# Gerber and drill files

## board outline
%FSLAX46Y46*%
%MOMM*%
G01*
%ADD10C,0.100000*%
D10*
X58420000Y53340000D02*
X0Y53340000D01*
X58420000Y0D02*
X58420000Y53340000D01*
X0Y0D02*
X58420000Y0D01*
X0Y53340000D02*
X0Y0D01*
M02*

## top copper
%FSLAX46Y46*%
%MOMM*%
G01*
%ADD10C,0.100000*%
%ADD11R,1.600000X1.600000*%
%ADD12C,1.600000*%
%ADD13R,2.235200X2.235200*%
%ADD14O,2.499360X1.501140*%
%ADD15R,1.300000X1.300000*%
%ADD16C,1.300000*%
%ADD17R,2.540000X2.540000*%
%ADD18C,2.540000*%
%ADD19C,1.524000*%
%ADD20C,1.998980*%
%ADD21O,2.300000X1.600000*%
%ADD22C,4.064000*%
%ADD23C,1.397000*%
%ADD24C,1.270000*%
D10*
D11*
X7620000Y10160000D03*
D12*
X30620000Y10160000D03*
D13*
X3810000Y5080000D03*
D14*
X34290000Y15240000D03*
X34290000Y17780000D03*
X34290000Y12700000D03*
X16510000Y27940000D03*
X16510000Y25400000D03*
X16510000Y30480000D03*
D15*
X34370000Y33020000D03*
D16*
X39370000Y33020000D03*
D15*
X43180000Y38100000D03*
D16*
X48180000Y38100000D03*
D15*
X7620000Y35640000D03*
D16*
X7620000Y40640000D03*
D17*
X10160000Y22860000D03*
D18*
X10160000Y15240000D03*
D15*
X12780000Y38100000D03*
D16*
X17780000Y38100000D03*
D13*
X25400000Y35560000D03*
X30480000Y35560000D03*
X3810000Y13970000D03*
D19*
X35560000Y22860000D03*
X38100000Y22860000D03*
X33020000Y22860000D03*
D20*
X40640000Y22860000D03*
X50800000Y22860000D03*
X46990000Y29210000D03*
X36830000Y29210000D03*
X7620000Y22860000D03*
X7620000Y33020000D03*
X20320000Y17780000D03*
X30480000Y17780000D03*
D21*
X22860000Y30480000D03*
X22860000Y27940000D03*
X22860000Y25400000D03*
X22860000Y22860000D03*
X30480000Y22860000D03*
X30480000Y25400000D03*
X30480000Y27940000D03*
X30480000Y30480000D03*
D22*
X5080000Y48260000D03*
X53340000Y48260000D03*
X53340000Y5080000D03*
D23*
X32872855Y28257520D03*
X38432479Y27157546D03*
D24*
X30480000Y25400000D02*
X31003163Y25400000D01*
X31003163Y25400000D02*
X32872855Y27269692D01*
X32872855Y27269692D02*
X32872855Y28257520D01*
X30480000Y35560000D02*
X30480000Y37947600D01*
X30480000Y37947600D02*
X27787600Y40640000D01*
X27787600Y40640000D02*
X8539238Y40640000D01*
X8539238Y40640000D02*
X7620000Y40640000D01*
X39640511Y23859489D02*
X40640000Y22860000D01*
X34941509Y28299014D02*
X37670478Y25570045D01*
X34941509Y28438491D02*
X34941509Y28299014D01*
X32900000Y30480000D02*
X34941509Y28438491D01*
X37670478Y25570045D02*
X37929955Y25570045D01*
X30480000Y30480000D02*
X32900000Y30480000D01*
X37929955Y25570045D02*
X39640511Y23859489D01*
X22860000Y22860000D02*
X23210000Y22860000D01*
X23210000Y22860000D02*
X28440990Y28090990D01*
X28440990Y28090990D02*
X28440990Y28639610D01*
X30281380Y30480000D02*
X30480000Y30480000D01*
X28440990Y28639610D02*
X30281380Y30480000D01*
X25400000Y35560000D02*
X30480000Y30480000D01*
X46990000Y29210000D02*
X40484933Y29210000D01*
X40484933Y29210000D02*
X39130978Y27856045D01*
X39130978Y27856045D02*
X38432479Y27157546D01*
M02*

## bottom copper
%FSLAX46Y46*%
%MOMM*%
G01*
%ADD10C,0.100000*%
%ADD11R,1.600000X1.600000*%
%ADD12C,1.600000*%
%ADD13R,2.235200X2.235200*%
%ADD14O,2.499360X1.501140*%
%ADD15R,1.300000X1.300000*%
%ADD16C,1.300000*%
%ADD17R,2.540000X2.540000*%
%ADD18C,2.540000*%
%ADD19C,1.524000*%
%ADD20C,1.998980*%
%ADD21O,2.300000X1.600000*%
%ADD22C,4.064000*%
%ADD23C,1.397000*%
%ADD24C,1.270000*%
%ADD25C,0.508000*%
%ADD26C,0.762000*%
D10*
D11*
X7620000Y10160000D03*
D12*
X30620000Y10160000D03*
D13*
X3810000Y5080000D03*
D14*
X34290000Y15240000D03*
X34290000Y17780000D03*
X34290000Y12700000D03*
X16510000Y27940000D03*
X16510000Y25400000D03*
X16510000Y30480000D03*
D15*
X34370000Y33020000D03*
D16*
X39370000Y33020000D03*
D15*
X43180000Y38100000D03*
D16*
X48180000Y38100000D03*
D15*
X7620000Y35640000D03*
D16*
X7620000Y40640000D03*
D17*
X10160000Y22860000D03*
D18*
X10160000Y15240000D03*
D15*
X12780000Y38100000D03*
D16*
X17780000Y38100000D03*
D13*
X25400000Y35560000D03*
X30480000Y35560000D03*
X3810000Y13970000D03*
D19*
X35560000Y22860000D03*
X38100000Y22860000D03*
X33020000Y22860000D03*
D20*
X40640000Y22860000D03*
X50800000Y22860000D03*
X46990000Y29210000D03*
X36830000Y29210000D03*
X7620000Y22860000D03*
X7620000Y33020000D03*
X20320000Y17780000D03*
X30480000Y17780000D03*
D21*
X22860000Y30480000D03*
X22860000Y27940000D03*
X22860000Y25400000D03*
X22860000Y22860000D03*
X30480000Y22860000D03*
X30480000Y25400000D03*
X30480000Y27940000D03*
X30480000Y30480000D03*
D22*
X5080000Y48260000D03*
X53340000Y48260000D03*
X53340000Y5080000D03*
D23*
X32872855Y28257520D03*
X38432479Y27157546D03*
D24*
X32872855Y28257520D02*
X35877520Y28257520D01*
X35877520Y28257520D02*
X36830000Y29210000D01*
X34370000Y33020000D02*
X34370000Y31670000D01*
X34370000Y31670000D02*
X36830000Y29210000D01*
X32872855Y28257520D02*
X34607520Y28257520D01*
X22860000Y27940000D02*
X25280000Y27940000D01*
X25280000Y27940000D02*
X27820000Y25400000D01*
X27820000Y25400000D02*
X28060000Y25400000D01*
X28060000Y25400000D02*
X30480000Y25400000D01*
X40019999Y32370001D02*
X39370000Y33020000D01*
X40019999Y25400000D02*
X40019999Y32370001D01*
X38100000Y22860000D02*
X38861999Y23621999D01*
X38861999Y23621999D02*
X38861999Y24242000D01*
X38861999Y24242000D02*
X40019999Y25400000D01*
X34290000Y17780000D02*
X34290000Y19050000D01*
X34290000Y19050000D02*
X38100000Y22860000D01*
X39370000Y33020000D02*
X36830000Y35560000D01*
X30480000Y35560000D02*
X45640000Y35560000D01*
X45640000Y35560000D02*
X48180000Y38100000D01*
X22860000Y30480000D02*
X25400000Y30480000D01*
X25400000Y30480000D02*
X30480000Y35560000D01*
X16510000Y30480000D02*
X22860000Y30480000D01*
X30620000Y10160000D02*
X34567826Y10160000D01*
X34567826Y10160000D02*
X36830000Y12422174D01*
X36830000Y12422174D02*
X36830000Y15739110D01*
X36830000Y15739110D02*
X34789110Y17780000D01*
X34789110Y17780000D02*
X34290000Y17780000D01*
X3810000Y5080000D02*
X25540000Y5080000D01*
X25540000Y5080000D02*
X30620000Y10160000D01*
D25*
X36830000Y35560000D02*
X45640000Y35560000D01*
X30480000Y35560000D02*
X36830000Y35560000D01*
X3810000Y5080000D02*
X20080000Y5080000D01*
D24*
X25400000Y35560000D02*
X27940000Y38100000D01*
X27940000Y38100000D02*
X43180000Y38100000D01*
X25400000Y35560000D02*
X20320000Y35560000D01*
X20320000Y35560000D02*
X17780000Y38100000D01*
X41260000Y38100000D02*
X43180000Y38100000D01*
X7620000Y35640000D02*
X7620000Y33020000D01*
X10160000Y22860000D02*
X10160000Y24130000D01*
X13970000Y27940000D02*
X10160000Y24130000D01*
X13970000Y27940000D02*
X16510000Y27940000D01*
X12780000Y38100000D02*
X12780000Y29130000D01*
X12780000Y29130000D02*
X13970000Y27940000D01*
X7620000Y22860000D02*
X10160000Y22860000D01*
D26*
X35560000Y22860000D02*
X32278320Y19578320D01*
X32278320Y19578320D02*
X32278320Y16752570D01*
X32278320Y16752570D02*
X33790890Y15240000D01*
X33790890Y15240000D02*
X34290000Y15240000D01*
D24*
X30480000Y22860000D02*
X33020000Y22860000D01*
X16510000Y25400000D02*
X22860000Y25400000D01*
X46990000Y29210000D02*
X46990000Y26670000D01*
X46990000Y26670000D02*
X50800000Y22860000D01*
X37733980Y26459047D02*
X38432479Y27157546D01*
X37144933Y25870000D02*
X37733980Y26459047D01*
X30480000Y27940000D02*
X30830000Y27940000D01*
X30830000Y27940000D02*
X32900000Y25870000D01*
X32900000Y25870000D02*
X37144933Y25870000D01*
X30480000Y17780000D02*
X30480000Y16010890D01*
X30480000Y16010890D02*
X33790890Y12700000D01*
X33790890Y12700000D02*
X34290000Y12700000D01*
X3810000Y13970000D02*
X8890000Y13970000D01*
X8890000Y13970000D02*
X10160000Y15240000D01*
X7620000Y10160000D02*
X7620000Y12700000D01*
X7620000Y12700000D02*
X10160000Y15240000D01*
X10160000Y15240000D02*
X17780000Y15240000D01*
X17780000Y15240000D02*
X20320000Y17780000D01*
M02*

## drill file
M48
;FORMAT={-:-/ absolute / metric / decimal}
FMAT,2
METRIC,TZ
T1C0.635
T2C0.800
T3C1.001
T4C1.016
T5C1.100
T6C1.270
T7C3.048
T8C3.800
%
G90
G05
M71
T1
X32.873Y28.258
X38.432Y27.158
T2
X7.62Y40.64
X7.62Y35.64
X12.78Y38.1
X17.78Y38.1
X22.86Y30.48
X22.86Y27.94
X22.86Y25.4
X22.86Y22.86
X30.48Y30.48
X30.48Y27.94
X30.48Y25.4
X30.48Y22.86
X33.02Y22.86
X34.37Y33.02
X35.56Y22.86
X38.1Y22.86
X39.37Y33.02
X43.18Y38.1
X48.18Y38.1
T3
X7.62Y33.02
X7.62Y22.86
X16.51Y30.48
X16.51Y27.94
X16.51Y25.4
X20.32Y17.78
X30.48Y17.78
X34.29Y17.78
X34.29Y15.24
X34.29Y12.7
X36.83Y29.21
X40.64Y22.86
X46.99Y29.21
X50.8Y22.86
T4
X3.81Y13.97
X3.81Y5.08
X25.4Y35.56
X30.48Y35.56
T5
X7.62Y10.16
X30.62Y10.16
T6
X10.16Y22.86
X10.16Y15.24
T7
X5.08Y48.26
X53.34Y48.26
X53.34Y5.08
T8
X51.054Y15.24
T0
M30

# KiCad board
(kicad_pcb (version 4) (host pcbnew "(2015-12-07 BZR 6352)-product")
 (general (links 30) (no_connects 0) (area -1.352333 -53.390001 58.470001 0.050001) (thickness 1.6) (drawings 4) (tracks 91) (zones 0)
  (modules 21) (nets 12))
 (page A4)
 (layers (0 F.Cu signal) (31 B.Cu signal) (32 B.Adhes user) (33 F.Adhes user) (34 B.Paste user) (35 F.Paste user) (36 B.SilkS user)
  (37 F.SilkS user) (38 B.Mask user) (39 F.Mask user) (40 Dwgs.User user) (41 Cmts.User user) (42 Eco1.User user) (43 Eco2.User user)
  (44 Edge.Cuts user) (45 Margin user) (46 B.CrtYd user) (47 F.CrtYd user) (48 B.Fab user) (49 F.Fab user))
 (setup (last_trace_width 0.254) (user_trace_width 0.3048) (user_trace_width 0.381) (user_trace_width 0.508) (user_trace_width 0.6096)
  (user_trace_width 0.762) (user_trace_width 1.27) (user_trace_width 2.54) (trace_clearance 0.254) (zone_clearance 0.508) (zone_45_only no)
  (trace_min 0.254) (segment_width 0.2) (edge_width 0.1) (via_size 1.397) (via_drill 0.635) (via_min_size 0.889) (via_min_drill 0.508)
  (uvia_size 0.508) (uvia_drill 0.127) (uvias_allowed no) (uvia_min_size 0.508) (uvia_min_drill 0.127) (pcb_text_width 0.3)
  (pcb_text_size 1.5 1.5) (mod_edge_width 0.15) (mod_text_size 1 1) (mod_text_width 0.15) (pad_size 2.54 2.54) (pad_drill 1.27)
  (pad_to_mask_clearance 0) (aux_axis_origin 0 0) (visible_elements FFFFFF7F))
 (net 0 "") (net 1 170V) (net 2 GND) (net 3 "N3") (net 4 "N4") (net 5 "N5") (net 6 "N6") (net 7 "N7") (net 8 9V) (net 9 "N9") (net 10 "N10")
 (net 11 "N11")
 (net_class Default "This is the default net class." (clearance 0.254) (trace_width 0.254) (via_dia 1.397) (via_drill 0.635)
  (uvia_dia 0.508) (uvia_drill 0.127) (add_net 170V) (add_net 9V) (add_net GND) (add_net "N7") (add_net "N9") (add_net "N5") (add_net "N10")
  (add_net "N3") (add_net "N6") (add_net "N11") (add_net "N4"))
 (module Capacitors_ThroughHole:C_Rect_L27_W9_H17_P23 (layer F.Cu) (at 7.62 -10.16)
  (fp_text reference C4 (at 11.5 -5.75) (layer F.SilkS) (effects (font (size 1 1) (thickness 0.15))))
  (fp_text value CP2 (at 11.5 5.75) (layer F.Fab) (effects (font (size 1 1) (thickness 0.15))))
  (pad 1 thru_hole rect (at 0 0) (size 1.6 1.6) (drill 1.1) (layers *.Cu *.Mask F.SilkS) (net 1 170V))
  (pad 2 thru_hole circle (at 23 0) (size 1.6 1.6) (drill 1.1) (layers *.Cu *.Mask F.SilkS) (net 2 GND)))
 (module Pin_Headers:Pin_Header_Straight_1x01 (layer F.Cu) (at 3.81 -5.08)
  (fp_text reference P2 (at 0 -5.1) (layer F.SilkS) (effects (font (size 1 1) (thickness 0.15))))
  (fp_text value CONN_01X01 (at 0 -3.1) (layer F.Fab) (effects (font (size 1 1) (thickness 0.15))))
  (pad 1 thru_hole rect (at 0 0) (size 2.2352 2.2352) (drill 1.016) (layers *.Cu *.Mask F.SilkS) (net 2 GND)))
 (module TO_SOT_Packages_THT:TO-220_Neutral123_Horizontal (layer F.Cu) (at 34.29 -15.24 270)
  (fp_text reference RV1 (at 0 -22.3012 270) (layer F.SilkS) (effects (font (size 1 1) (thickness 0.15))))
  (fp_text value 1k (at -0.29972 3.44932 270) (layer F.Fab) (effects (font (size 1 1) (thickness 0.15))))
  (pad 2 thru_hole oval (at 0 0) (size 2.49936 1.50114) (drill 1.00076) (layers *.Cu *.Mask F.SilkS) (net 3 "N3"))
  (pad 1 thru_hole oval (at -2.54 0) (size 2.49936 1.50114) (drill 1.00076) (layers *.Cu *.Mask F.SilkS) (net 2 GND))
  (pad 3 thru_hole oval (at 2.54 0) (size 2.49936 1.50114) (drill 1.00076) (layers *.Cu *.Mask F.SilkS) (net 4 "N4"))
  (pad "" np_thru_hole circle (at 0 -16.764) (size 3.79984 3.79984) (drill 3.79984) (layers *.Cu *.Mask F.SilkS)))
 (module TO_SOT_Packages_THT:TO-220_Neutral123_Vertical (layer F.Cu) (at 16.51 -27.94 90)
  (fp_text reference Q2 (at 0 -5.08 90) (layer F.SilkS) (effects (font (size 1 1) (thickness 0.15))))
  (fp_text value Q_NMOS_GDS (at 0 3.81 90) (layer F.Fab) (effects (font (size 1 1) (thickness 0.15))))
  (pad 2 thru_hole oval (at 0 0 180) (size 2.49936 1.50114) (drill 1.00076) (layers *.Cu *.Mask F.SilkS) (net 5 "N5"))
  (pad 1 thru_hole oval (at -2.54 0 180) (size 2.49936 1.50114) (drill 1.00076) (layers *.Cu *.Mask F.SilkS) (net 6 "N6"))
  (pad 3 thru_hole oval (at 2.54 0 180) (size 2.49936 1.50114) (drill 1.00076) (layers *.Cu *.Mask F.SilkS) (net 2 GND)))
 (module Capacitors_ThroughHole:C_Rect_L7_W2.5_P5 (layer F.Cu) (at 34.37 -33.02)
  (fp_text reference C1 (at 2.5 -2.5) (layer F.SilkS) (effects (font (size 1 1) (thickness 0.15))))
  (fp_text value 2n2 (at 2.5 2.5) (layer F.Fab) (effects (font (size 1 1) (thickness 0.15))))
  (pad 1 thru_hole rect (at 0 0) (size 1.3 1.3) (drill 0.8) (layers *.Cu *.Mask F.SilkS) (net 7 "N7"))
  (pad 2 thru_hole circle (at 5 0) (size 1.3 1.3) (drill 0.8) (layers *.Cu *.Mask F.SilkS) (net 2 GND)))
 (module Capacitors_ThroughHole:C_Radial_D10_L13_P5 (layer F.Cu) (at 43.18 -38.1)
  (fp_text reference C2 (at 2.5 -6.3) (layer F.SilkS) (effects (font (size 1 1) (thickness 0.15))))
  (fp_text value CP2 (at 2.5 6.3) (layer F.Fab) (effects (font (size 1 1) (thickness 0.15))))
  (pad 1 thru_hole rect (at 0 0) (size 1.3 1.3) (drill 0.8) (layers *.Cu *.Mask F.SilkS) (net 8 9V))
  (pad 2 thru_hole circle (at 5 0) (size 1.3 1.3) (drill 0.8) (layers *.Cu *.Mask F.SilkS) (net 2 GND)))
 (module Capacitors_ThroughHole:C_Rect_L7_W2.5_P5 (layer F.Cu) (at 7.62 -35.64 90)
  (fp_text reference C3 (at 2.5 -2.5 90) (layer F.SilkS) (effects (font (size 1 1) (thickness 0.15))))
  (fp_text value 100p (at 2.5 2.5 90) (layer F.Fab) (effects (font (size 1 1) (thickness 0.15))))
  (pad 1 thru_hole rect (at 0 0 90) (size 1.3 1.3) (drill 0.8) (layers *.Cu *.Mask F.SilkS) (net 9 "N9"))
  (pad 2 thru_hole circle (at 5 0 90) (size 1.3 1.3) (drill 0.8) (layers *.Cu *.Mask F.SilkS) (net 2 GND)))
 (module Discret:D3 (layer F.Cu) (at 10.16 -19.05 90)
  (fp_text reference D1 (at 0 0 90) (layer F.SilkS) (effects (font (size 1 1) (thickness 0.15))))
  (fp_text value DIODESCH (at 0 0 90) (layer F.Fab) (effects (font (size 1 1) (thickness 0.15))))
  (pad 1 thru_hole rect (at 3.81 0 90) (size 2.54 2.54) (drill 1.27) (layers *.Cu *.Mask F.SilkS) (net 5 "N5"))
  (pad 2 thru_hole circle (at -3.81 0 90) (size 2.54 2.54) (drill 1.27) (layers *.Cu *.Mask F.SilkS) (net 1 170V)))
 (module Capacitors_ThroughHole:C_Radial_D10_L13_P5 (layer F.Cu) (at 12.78 -38.1)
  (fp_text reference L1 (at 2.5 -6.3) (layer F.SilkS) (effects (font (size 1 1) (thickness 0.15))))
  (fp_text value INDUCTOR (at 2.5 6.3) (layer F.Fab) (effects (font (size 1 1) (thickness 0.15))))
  (pad 1 thru_hole rect (at 0 0) (size 1.3 1.3) (drill 0.8) (layers *.Cu *.Mask F.SilkS) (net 5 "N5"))
  (pad 2 thru_hole circle (at 5 0) (size 1.3 1.3) (drill 0.8) (layers *.Cu *.Mask F.SilkS) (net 8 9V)))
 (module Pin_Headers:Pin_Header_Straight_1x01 (layer F.Cu) (at 25.4 -35.56)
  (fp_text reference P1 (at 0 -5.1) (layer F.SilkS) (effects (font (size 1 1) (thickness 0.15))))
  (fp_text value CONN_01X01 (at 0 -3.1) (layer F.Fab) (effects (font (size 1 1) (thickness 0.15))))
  (pad 1 thru_hole rect (at 0 0) (size 2.2352 2.2352) (drill 1.016) (layers *.Cu *.Mask F.SilkS) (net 8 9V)))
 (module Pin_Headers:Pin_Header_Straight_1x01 (layer F.Cu) (at 30.48 -35.56)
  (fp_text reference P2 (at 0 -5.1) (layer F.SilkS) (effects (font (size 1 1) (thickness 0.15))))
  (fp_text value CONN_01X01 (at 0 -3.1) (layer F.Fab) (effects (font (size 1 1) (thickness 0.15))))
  (pad 1 thru_hole rect (at 0 0) (size 2.2352 2.2352) (drill 1.016) (layers *.Cu *.Mask F.SilkS) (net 2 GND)))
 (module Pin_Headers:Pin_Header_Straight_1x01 (layer F.Cu) (at 3.81 -13.97)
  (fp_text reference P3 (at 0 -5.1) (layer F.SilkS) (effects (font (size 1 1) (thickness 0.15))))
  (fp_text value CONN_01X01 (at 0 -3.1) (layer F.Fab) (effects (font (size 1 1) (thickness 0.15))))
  (pad 1 thru_hole rect (at 0 0) (size 2.2352 2.2352) (drill 1.016) (layers *.Cu *.Mask F.SilkS) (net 1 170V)))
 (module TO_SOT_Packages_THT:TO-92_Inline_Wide (layer F.Cu) (at 33.02 -22.86)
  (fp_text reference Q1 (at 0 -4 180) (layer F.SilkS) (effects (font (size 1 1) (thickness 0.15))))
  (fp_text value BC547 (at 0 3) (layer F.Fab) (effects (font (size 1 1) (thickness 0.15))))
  (pad 2 thru_hole circle (at 2.54 0 90) (size 1.524 1.524) (drill 0.8) (layers *.Cu *.Mask F.SilkS) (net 3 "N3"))
  (pad 3 thru_hole circle (at 5.08 0 90) (size 1.524 1.524) (drill 0.8) (layers *.Cu *.Mask F.SilkS) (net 2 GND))
  (pad 1 thru_hole circle (at 0 0 90) (size 1.524 1.524) (drill 0.8) (layers *.Cu *.Mask F.SilkS) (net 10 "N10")))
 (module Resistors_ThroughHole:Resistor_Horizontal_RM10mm (layer F.Cu) (at 45.72 -22.86)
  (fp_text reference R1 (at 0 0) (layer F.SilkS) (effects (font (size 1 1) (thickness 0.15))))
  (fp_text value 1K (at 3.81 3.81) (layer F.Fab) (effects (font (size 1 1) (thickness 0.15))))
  (pad 1 thru_hole circle (at -5.08 0) (size 1.99898 1.99898) (drill 1.00076) (layers *.Cu *.SilkS *.Mask) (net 8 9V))
  (pad 2 thru_hole circle (at 5.08 0) (size 1.99898 1.99898) (drill 1.00076) (layers *.Cu *.SilkS *.Mask) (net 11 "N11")))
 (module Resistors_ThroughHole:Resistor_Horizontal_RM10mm (layer F.Cu) (at 41.91 -29.21 180)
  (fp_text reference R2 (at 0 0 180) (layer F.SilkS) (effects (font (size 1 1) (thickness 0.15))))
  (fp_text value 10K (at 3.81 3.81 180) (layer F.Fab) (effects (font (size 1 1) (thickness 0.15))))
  (pad 1 thru_hole circle (at -5.08 0 180) (size 1.99898 1.99898) (drill 1.00076) (layers *.Cu *.SilkS *.Mask) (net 11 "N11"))
  (pad 2 thru_hole circle (at 5.08 0 180) (size 1.99898 1.99898) (drill 1.00076) (layers *.Cu *.SilkS *.Mask) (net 7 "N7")))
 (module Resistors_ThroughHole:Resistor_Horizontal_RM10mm (layer F.Cu) (at 7.62 -27.94 90)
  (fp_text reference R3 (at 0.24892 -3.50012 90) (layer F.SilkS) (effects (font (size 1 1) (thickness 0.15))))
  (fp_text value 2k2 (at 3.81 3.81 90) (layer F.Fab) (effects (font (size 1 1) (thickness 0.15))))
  (pad 1 thru_hole circle (at -5.08 0 90) (size 1.99898 1.99898) (drill 1.00076) (layers *.Cu *.SilkS *.Mask) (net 5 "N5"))
  (pad 2 thru_hole circle (at 5.08 0 90) (size 1.99898 1.99898) (drill 1.00076) (layers *.Cu *.SilkS *.Mask) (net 9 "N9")))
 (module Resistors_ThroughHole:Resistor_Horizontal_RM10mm (layer F.Cu) (at 25.4 -17.78)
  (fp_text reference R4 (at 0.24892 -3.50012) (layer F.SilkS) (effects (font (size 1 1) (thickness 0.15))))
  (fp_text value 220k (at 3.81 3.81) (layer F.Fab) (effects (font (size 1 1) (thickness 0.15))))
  (pad 1 thru_hole circle (at -5.08 0) (size 1.99898 1.99898) (drill 1.00076) (layers *.Cu *.SilkS *.Mask) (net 1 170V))
  (pad 2 thru_hole circle (at 5.08 0) (size 1.99898 1.99898) (drill 1.00076) (layers *.Cu *.SilkS *.Mask) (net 4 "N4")))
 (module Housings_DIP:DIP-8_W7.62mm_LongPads (layer F.Cu) (at 22.86 -30.48)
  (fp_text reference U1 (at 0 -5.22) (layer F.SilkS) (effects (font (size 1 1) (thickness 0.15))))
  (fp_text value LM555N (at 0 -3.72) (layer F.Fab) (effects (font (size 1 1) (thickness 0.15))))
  (pad 1 thru_hole oval (at 0 0) (size 2.3 1.6) (drill 0.8) (layers *.Cu *.Mask F.SilkS) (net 2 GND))
  (pad 2 thru_hole oval (at 0 2.54) (size 2.3 1.6) (drill 0.8) (layers *.Cu *.Mask F.SilkS) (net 7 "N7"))
  (pad 3 thru_hole oval (at 0 5.08) (size 2.3 1.6) (drill 0.8) (layers *.Cu *.Mask F.SilkS) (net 6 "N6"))
  (pad 4 thru_hole oval (at 0 7.62) (size 2.3 1.6) (drill 0.8) (layers *.Cu *.Mask F.SilkS) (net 8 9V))
  (pad 5 thru_hole oval (at 7.62 7.62) (size 2.3 1.6) (drill 0.8) (layers *.Cu *.Mask F.SilkS) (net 10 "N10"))
  (pad 6 thru_hole oval (at 7.62 5.08) (size 2.3 1.6) (drill 0.8) (layers *.Cu *.Mask F.SilkS) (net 7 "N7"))
  (pad 7 thru_hole oval (at 7.62 2.54) (size 2.3 1.6) (drill 0.8) (layers *.Cu *.Mask F.SilkS) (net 11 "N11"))
  (pad 8 thru_hole oval (at 7.62 0) (size 2.3 1.6) (drill 0.8) (layers *.Cu *.Mask F.SilkS) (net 8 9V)))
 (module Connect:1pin (layer F.Cu) (at 5.08 -48.26)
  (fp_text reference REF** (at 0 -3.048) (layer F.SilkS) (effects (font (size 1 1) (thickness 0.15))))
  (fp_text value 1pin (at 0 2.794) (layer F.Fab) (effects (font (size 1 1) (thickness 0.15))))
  (pad 1 thru_hole circle (at 0 0) (size 4.064 4.064) (drill 3.048) (layers *.Cu *.Mask F.SilkS)))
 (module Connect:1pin (layer F.Cu) (at 53.34 -48.26)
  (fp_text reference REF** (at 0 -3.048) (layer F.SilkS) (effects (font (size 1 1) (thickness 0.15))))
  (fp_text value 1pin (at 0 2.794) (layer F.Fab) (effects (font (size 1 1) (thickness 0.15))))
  (pad 1 thru_hole circle (at 0 0) (size 4.064 4.064) (drill 3.048) (layers *.Cu *.Mask F.SilkS)))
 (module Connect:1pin (layer F.Cu) (at 53.34 -5.08)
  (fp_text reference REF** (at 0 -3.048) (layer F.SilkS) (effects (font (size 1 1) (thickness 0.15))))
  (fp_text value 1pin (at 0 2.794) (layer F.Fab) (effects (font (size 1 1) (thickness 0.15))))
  (pad 1 thru_hole circle (at 0 0) (size 4.064 4.064) (drill 3.048) (layers *.Cu *.Mask F.SilkS)))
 (gr_line (start 58.42 -53.34) (end 0 -53.34) (layer Edge.Cuts) (width 0.1))
 (gr_line (start 58.42 0) (end 58.42 -53.34) (layer Edge.Cuts) (width 0.1))
 (gr_line (start 0 0) (end 58.42 0) (layer Edge.Cuts) (width 0.1))
 (gr_line (start 0 -53.34) (end 0 0) (layer Edge.Cuts) (width 0.1))
 (segment (start 32.872855 -28.25752) (end 35.87752 -28.25752) (width 1.27) (layer B.Cu) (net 7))
 (segment (start 35.87752 -28.25752) (end 36.83 -29.21) (width 1.27) (layer B.Cu) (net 7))
 (segment (start 34.37 -33.02) (end 34.37 -31.67) (width 1.27) (layer B.Cu) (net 7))
 (segment (start 34.37 -31.67) (end 36.83 -29.21) (width 1.27) (layer B.Cu) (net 7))
 (segment (start 30.48 -25.4) (end 31.003163 -25.4) (width 1.27) (layer F.Cu) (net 7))
 (segment (start 31.003163 -25.4) (end 32.872855 -27.269692) (width 1.27) (layer F.Cu) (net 7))
 (segment (start 32.872855 -27.269692) (end 32.872855 -28.25752) (width 1.27) (layer F.Cu) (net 7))
 (segment (start 32.872855 -28.25752) (end 34.60752 -28.25752) (width 1.27) (layer B.Cu) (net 7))
 (via (at 32.872855 -28.25752) (size 1.397) (drill 0.635) (layers F.Cu B.Cu) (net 7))
 (segment (start 22.86 -27.94) (end 25.28 -27.94) (width 1.27) (layer B.Cu) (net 7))
 (segment (start 25.28 -27.94) (end 27.82 -25.4) (width 1.27) (layer B.Cu) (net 7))
 (segment (start 27.82 -25.4) (end 28.06 -25.4) (width 1.27) (layer B.Cu) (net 7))
 (segment (start 28.06 -25.4) (end 30.48 -25.4) (width 1.27) (layer B.Cu) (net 7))
 (segment (start 40.019999 -32.370001) (end 39.37 -33.02) (width 1.27) (layer B.Cu) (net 2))
 (segment (start 40.019999 -25.4) (end 40.019999 -32.370001) (width 1.27) (layer B.Cu) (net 2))
 (segment (start 38.1 -22.86) (end 38.861999 -23.621999) (width 1.27) (layer B.Cu) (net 2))
 (segment (start 38.861999 -23.621999) (end 38.861999 -24.242) (width 1.27) (layer B.Cu) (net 2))
 (segment (start 38.861999 -24.242) (end 40.019999 -25.4) (width 1.27) (layer B.Cu) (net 2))
 (segment (start 30.48 -35.56) (end 30.48 -37.9476) (width 1.27) (layer F.Cu) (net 2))
 (segment (start 30.48 -37.9476) (end 27.7876 -40.64) (width 1.27) (layer F.Cu) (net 2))
 (segment (start 27.7876 -40.64) (end 8.539238 -40.64) (width 1.27) (layer F.Cu) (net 2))
 (segment (start 8.539238 -40.64) (end 7.62 -40.64) (width 1.27) (layer F.Cu) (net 2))
 (segment (start 34.29 -17.78) (end 34.29 -19.05) (width 1.27) (layer B.Cu) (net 2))
 (segment (start 34.29 -19.05) (end 38.1 -22.86) (width 1.27) (layer B.Cu) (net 2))
 (segment (start 39.37 -33.02) (end 36.83 -35.56) (width 1.27) (layer B.Cu) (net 2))
 (segment (start 30.48 -35.56) (end 45.64 -35.56) (width 1.27) (layer B.Cu) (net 2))
 (segment (start 45.64 -35.56) (end 48.18 -38.1) (width 1.27) (layer B.Cu) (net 2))
 (segment (start 22.86 -30.48) (end 25.4 -30.48) (width 1.27) (layer B.Cu) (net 2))
 (segment (start 25.4 -30.48) (end 30.48 -35.56) (width 1.27) (layer B.Cu) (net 2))
 (segment (start 16.51 -30.48) (end 22.86 -30.48) (width 1.27) (layer B.Cu) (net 2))
 (segment (start 30.62 -10.16) (end 34.567826 -10.16) (width 1.27) (layer B.Cu) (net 2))
 (segment (start 34.567826 -10.16) (end 36.83 -12.422174) (width 1.27) (layer B.Cu) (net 2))
 (segment (start 36.83 -12.422174) (end 36.83 -15.73911) (width 1.27) (layer B.Cu) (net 2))
 (segment (start 36.83 -15.73911) (end 34.78911 -17.78) (width 1.27) (layer B.Cu) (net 2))
 (segment (start 34.78911 -17.78) (end 34.29 -17.78) (width 1.27) (layer B.Cu) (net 2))
 (segment (start 3.81 -5.08) (end 25.54 -5.08) (width 1.27) (layer B.Cu) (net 2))
 (segment (start 25.54 -5.08) (end 30.62 -10.16) (width 1.27) (layer B.Cu) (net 2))
 (segment (start 36.83 -35.56) (end 45.64 -35.56) (width 0.508) (layer B.Cu) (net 2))
 (segment (start 30.48 -35.56) (end 36.83 -35.56) (width 0.508) (layer B.Cu) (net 2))
 (segment (start 3.81 -5.08) (end 20.08 -5.08) (width 0.508) (layer B.Cu) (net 2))
 (segment (start 39.640511 -23.859489) (end 40.64 -22.86) (width 1.27) (layer F.Cu) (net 8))
 (segment (start 34.941509 -28.299014) (end 37.670478 -25.570045) (width 1.27) (layer F.Cu) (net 8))
 (segment (start 34.941509 -28.438491) (end 34.941509 -28.299014) (width 1.27) (layer F.Cu) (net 8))
 (segment (start 32.9 -30.48) (end 34.941509 -28.438491) (width 1.27) (layer F.Cu) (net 8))
 (segment (start 37.670478 -25.570045) (end 37.929955 -25.570045) (width 1.27) (layer F.Cu) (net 8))
 (segment (start 30.48 -30.48) (end 32.9 -30.48) (width 1.27) (layer F.Cu) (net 8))
 (segment (start 37.929955 -25.570045) (end 39.640511 -23.859489) (width 1.27) (layer F.Cu) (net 8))
 (segment (start 22.86 -22.86) (end 23.21 -22.86) (width 1.27) (layer F.Cu) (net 8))
 (segment (start 23.21 -22.86) (end 28.44099 -28.09099) (width 1.27) (layer F.Cu) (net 8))
 (segment (start 28.44099 -28.09099) (end 28.44099 -28.63961) (width 1.27) (layer F.Cu) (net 8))
 (segment (start 30.28138 -30.48) (end 30.48 -30.48) (width 1.27) (layer F.Cu) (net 8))
 (segment (start 28.44099 -28.63961) (end 30.28138 -30.48) (width 1.27) (layer F.Cu) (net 8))
 (segment (start 25.4 -35.56) (end 30.48 -30.48) (width 1.27) (layer F.Cu) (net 8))
 (segment (start 25.4 -35.56) (end 27.94 -38.1) (width 1.27) (layer B.Cu) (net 8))
 (segment (start 27.94 -38.1) (end 43.18 -38.1) (width 1.27) (layer B.Cu) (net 8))
 (segment (start 25.4 -35.56) (end 20.32 -35.56) (width 1.27) (layer B.Cu) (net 8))
 (segment (start 20.32 -35.56) (end 17.78 -38.1) (width 1.27) (layer B.Cu) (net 8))
 (segment (start 41.26 -38.1) (end 43.18 -38.1) (width 1.27) (layer B.Cu) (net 8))
 (segment (start 7.62 -35.64) (end 7.62 -33.02) (width 1.27) (layer B.Cu) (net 9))
 (segment (start 10.16 -22.86) (end 10.16 -24.13) (width 1.27) (layer B.Cu) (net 5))
 (segment (start 13.97 -27.94) (end 10.16 -24.13) (width 1.27) (layer B.Cu) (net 5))
 (segment (start 13.97 -27.94) (end 16.51 -27.94) (width 1.27) (layer B.Cu) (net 5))
 (segment (start 12.78 -38.1) (end 12.78 -29.13) (width 1.27) (layer B.Cu) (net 5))
 (segment (start 12.78 -29.13) (end 13.97 -27.94) (width 1.27) (layer B.Cu) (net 5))
 (segment (start 7.62 -22.86) (end 10.16 -22.86) (width 1.27) (layer B.Cu) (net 5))
 (segment (start 35.56 -22.86) (end 32.27832 -19.57832) (width 0.762) (layer B.Cu) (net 3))
 (segment (start 32.27832 -19.57832) (end 32.27832 -16.75257) (width 0.762) (layer B.Cu) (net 3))
 (segment (start 32.27832 -16.75257) (end 33.79089 -15.24) (width 0.762) (layer B.Cu) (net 3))
 (segment (start 33.79089 -15.24) (end 34.29 -15.24) (width 0.762) (layer B.Cu) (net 3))
 (segment (start 30.48 -22.86) (end 33.02 -22.86) (width 1.27) (layer B.Cu) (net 10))
 (segment (start 16.51 -25.4) (end 22.86 -25.4) (width 1.27) (layer B.Cu) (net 6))
 (segment (start 46.99 -29.21) (end 40.484933 -29.21) (width 1.27) (layer F.Cu) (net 11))
 (segment (start 40.484933 -29.21) (end 39.130978 -27.856045) (width 1.27) (layer F.Cu) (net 11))
 (segment (start 39.130978 -27.856045) (end 38.432479 -27.157546) (width 1.27) (layer F.Cu) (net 11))
 (segment (start 46.99 -29.21) (end 46.99 -26.67) (width 1.27) (layer B.Cu) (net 11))
 (segment (start 46.99 -26.67) (end 50.8 -22.86) (width 1.27) (layer B.Cu) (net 11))
 (segment (start 37.73398 -26.459047) (end 38.432479 -27.157546) (width 1.27) (layer B.Cu) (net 11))
 (segment (start 37.144933 -25.87) (end 37.73398 -26.459047) (width 1.27) (layer B.Cu) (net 11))
 (segment (start 30.48 -27.94) (end 30.83 -27.94) (width 1.27) (layer B.Cu) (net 11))
 (segment (start 30.83 -27.94) (end 32.9 -25.87) (width 1.27) (layer B.Cu) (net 11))
 (via (at 38.432479 -27.157546) (size 1.397) (drill 0.635) (layers F.Cu B.Cu) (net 11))
 (segment (start 32.9 -25.87) (end 37.144933 -25.87) (width 1.27) (layer B.Cu) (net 11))
 (segment (start 30.48 -17.78) (end 30.48 -16.01089) (width 1.27) (layer B.Cu) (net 4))
 (segment (start 30.48 -16.01089) (end 33.79089 -12.7) (width 1.27) (layer B.Cu) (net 4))
 (segment (start 33.79089 -12.7) (end 34.29 -12.7) (width 1.27) (layer B.Cu) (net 4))
 (segment (start 3.81 -13.97) (end 8.89 -13.97) (width 1.27) (layer B.Cu) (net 1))
 (segment (start 8.89 -13.97) (end 10.16 -15.24) (width 1.27) (layer B.Cu) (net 1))
 (segment (start 7.62 -10.16) (end 7.62 -12.7) (width 1.27) (layer B.Cu) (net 1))
 (segment (start 7.62 -12.7) (end 10.16 -15.24) (width 1.27) (layer B.Cu) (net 1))
 (segment (start 10.16 -15.24) (end 17.78 -15.24) (width 1.27) (layer B.Cu) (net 1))
 (segment (start 17.78 -15.24) (end 20.32 -17.78) (width 1.27) (layer B.Cu) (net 1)))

